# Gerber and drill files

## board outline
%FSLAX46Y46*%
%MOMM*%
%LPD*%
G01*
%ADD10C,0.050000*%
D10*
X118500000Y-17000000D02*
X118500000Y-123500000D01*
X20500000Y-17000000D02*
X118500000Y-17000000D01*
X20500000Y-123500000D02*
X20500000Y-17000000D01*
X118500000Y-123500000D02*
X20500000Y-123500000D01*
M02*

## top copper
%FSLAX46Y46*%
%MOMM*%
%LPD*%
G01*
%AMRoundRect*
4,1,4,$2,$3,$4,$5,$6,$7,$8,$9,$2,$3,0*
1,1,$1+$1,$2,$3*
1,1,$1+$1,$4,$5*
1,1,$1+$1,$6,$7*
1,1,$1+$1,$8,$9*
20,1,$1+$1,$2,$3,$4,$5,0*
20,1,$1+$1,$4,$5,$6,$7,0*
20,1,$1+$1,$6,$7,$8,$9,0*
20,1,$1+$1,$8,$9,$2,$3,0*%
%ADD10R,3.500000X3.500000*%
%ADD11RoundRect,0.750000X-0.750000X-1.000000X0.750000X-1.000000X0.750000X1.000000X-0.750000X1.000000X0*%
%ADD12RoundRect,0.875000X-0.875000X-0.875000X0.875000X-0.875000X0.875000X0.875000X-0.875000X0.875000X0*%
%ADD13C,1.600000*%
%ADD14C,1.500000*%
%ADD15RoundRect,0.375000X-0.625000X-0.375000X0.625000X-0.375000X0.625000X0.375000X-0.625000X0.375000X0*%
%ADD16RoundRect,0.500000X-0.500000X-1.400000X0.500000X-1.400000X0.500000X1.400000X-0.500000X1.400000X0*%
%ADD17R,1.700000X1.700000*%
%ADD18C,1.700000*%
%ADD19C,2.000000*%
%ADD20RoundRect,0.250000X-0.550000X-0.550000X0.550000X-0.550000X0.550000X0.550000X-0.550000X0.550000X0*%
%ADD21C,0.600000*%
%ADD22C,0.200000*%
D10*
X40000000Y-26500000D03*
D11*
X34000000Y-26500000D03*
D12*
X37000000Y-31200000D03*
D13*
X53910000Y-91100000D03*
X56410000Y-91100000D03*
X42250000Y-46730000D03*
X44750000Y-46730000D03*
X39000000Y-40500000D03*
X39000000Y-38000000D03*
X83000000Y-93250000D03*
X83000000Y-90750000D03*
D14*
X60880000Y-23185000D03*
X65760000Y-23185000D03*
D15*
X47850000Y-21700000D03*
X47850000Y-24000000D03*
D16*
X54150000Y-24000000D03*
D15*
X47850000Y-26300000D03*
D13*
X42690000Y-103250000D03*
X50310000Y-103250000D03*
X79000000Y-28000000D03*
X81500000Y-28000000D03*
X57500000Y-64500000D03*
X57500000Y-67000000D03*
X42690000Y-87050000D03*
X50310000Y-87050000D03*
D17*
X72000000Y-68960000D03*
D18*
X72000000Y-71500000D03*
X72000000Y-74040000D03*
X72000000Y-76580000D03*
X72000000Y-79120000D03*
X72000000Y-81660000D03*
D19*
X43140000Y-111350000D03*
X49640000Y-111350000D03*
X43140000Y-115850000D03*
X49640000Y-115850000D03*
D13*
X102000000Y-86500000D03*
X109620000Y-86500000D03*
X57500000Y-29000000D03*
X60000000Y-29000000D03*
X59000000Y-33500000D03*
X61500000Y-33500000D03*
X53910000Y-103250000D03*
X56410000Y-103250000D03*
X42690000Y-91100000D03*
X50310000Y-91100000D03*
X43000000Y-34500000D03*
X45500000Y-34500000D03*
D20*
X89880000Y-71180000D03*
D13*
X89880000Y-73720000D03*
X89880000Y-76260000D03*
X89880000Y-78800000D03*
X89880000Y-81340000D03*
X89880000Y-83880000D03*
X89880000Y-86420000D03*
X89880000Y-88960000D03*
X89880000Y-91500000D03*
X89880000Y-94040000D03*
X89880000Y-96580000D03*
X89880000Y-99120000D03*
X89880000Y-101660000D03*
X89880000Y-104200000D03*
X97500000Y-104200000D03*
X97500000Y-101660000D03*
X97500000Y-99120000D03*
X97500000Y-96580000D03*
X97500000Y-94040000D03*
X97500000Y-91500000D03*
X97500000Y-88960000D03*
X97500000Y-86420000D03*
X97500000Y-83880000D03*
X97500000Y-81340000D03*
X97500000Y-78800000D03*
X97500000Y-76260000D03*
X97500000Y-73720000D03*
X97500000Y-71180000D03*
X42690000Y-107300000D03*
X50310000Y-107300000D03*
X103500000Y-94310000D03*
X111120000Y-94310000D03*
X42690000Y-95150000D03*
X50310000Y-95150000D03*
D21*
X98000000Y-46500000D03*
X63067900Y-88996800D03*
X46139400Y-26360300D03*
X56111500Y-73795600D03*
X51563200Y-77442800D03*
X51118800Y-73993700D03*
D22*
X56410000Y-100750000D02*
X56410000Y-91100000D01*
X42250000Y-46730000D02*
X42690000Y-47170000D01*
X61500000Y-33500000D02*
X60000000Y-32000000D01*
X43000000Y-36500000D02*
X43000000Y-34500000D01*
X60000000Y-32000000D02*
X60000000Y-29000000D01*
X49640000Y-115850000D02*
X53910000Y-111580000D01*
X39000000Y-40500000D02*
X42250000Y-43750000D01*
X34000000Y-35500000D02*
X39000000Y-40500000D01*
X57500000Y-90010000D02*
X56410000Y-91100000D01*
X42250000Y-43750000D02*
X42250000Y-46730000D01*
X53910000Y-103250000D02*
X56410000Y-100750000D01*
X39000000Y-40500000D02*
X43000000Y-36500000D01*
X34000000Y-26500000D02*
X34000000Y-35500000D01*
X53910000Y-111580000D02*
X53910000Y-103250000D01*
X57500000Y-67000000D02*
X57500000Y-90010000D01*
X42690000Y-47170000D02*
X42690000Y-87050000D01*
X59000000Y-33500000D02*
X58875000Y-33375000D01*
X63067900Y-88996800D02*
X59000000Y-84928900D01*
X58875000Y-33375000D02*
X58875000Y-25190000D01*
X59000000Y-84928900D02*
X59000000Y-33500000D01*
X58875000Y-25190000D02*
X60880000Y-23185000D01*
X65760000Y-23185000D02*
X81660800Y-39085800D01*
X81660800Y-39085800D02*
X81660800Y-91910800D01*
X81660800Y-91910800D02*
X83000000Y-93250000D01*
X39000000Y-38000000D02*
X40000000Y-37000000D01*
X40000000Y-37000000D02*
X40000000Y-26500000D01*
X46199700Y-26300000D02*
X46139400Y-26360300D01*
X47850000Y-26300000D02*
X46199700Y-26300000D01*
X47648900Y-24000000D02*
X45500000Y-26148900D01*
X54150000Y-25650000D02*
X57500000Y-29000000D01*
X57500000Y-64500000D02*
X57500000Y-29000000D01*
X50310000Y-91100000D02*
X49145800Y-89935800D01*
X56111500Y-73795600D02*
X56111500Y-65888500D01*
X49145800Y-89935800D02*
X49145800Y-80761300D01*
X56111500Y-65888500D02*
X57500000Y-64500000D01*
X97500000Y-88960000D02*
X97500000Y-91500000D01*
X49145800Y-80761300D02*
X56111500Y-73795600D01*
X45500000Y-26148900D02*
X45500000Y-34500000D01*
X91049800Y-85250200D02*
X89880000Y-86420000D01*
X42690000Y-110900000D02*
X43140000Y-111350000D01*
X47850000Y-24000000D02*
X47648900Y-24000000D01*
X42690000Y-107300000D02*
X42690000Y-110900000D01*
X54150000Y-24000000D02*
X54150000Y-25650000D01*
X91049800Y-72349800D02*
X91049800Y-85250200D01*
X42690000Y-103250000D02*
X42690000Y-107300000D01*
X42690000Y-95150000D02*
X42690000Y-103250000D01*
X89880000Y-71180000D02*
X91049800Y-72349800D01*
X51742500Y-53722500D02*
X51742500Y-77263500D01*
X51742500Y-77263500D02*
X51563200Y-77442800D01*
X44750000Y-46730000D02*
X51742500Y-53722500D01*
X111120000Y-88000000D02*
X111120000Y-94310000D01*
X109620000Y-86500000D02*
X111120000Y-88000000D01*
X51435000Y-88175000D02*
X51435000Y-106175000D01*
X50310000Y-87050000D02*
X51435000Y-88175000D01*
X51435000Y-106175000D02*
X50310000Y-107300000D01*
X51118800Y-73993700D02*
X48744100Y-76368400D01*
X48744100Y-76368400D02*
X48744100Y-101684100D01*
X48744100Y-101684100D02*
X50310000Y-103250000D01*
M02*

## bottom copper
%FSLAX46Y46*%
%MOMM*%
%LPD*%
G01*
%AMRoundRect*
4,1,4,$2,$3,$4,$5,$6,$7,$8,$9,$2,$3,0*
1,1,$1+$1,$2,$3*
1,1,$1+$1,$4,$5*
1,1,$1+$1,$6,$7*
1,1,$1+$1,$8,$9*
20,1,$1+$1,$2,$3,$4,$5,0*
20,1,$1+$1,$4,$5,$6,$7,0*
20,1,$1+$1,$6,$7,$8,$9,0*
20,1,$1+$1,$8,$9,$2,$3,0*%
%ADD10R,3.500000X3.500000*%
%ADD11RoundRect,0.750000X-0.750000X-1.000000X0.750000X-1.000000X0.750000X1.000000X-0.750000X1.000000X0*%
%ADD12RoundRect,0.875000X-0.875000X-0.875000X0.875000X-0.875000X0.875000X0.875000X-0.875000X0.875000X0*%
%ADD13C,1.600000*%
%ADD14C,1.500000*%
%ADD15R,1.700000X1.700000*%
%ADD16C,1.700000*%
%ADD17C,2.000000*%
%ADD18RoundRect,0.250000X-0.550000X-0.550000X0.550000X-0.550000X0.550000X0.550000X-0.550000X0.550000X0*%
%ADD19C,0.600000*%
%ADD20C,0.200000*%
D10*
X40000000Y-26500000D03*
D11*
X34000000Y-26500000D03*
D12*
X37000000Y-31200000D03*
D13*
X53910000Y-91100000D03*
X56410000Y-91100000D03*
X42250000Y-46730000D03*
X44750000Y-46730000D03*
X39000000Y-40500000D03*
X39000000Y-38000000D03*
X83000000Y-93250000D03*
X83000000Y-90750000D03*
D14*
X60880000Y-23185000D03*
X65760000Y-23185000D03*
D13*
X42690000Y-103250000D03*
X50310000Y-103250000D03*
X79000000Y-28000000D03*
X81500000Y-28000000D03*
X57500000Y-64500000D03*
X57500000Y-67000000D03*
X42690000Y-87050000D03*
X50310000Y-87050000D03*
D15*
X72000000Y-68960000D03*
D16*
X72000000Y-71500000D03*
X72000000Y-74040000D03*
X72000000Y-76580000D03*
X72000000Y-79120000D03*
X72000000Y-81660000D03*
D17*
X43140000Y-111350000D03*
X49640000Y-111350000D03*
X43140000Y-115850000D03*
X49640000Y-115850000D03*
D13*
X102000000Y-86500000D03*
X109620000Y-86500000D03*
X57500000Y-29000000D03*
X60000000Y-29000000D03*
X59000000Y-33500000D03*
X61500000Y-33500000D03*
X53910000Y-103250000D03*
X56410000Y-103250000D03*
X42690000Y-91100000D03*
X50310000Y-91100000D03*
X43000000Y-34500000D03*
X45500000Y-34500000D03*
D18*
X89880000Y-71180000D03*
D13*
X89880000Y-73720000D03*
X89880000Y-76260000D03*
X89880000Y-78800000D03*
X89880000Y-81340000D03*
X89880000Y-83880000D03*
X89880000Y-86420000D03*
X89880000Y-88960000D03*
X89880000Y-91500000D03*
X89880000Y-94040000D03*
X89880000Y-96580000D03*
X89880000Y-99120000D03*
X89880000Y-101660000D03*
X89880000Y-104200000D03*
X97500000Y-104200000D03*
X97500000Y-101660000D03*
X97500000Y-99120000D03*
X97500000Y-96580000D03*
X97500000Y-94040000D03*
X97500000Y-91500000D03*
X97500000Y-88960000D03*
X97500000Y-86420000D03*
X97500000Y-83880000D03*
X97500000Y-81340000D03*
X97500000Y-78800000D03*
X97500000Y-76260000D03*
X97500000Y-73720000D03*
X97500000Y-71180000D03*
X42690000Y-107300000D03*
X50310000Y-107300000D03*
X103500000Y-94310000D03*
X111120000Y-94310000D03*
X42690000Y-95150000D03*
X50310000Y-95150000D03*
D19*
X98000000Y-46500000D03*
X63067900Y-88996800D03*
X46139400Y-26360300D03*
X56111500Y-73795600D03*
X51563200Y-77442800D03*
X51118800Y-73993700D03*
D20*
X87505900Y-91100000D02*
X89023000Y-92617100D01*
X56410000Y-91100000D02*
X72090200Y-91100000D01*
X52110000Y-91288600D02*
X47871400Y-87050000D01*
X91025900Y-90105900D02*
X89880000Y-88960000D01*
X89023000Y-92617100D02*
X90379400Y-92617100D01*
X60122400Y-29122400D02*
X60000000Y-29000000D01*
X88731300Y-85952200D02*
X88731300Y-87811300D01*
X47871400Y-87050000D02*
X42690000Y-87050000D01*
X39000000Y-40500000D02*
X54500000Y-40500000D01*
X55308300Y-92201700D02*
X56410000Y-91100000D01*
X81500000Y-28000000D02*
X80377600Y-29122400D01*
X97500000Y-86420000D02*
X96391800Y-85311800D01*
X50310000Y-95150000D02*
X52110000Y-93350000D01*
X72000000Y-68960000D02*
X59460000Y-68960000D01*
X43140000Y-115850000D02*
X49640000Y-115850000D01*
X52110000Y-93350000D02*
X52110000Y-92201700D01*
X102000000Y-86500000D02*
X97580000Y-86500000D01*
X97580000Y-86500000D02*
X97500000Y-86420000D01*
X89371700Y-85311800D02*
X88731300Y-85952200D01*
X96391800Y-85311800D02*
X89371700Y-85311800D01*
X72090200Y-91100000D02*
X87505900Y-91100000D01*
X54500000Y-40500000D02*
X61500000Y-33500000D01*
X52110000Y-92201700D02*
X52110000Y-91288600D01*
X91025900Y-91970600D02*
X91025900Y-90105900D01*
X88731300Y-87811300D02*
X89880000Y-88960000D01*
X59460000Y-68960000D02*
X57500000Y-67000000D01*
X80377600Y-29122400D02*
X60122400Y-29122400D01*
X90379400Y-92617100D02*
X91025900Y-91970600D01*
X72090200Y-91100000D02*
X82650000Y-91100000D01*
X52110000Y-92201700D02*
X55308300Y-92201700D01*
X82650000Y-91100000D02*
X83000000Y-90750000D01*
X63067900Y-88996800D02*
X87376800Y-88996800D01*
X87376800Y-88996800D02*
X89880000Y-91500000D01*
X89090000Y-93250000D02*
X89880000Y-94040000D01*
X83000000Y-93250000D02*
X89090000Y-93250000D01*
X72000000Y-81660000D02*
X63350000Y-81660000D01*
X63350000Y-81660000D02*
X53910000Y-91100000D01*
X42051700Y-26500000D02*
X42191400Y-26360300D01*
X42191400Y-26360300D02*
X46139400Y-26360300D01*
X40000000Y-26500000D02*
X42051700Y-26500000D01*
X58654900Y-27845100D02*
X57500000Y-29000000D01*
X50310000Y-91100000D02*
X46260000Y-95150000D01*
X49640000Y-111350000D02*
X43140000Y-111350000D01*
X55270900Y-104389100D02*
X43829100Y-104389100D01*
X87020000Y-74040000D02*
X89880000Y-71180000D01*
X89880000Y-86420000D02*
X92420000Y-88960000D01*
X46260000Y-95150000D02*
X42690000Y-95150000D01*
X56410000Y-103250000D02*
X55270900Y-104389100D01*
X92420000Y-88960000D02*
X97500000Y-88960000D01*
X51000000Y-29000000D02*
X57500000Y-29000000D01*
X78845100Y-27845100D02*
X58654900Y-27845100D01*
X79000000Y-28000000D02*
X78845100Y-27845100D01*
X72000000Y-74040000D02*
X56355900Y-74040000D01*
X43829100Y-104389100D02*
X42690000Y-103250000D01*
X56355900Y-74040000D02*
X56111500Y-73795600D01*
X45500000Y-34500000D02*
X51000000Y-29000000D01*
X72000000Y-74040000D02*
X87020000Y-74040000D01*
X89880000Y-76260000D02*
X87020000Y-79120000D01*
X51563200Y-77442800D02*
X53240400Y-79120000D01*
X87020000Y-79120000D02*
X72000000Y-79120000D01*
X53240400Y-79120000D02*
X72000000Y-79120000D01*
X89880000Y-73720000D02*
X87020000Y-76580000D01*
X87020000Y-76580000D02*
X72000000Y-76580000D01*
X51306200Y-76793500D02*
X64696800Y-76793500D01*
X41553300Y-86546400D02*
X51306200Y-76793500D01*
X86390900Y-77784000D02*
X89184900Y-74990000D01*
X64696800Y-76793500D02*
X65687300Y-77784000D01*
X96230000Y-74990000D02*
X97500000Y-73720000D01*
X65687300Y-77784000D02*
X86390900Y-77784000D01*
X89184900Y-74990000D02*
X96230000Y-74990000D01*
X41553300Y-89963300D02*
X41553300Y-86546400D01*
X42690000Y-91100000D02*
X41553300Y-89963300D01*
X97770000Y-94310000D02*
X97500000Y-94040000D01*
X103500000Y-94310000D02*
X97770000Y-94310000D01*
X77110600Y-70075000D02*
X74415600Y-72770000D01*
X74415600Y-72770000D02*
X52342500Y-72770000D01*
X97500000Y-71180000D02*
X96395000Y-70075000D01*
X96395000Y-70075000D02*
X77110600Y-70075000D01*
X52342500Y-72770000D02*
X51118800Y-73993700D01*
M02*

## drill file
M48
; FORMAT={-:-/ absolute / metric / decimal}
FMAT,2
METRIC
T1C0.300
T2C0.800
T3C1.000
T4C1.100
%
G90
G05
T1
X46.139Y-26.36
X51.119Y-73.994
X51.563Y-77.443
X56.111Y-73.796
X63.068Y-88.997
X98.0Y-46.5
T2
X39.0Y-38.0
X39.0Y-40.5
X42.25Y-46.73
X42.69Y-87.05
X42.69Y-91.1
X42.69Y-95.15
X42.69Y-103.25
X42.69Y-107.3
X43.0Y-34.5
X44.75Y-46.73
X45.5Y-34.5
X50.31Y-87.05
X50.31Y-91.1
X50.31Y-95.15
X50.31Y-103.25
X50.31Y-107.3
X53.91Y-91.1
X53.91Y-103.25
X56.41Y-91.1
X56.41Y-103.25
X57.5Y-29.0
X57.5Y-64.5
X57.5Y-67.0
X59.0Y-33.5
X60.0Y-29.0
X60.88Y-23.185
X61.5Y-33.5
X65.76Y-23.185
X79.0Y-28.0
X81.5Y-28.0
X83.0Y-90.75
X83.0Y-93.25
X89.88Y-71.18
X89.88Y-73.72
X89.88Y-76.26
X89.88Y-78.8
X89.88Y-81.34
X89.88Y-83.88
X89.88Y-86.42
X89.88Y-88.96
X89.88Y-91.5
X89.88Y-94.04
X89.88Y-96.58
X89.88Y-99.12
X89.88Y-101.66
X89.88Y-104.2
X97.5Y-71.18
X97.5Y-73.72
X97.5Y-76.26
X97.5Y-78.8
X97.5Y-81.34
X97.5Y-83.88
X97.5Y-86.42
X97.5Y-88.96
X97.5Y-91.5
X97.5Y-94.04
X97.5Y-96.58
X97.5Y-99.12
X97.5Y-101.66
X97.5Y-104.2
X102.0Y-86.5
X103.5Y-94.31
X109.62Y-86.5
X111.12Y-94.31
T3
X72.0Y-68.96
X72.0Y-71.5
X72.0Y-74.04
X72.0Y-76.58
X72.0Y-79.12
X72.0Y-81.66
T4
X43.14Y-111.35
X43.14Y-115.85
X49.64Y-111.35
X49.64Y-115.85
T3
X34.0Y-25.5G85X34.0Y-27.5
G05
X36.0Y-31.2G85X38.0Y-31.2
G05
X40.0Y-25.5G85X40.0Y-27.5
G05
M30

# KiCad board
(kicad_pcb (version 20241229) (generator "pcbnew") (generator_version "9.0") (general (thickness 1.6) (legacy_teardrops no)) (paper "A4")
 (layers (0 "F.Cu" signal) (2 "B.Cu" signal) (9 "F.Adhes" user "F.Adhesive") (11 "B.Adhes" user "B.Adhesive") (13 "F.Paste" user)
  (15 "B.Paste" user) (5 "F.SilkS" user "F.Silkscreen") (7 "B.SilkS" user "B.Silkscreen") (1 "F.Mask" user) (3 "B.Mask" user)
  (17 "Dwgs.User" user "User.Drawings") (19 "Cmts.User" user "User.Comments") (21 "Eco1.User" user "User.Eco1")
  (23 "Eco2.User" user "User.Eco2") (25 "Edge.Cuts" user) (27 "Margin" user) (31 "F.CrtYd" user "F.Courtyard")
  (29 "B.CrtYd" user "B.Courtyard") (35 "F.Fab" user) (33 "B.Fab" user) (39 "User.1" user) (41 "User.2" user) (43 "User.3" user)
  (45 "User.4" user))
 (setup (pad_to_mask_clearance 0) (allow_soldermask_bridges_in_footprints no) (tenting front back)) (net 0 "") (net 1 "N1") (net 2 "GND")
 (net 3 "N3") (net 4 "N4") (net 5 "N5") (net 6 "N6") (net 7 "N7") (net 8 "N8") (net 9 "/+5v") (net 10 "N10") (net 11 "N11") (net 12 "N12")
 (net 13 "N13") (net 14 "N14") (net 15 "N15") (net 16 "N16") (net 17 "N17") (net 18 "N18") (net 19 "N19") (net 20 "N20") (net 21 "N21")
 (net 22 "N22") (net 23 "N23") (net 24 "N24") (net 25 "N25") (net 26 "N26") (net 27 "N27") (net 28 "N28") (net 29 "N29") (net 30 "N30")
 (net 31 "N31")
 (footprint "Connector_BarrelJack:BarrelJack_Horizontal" (layer "F.Cu") (at 40 26.5)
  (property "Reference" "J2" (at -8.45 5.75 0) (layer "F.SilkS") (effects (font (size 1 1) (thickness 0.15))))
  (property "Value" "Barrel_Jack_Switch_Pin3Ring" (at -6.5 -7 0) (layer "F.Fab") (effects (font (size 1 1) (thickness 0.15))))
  (pad "1" thru_hole rect (at 0 0) (size 3.5 3.5) (drill oval 1 3) (layers "*.Cu" "*.Mask") (remove_unused_layers no) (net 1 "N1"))
  (pad "2" thru_hole roundrect (at -6 0) (size 3 3.5) (drill oval 1 3) (layers "*.Cu" "*.Mask") (remove_unused_layers no)
   (roundrect_rratio 0.25) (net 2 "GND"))
  (pad "3" thru_hole roundrect (at -3 4.7) (size 3.5 3.5) (drill oval 3 1) (layers "*.Cu" "*.Mask") (remove_unused_layers no)
   (roundrect_rratio 0.25) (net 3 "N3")))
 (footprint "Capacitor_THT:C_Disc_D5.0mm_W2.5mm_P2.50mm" (layer "F.Cu") (at 53.91 91.1)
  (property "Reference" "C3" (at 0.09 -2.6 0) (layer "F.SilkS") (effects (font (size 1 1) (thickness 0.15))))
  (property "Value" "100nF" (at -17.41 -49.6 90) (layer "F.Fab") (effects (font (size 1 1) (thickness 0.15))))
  (pad "1" thru_hole circle (at 0 0) (size 1.6 1.6) (drill 0.8) (layers "*.Cu" "*.Mask") (remove_unused_layers no) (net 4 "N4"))
  (pad "2" thru_hole circle (at 2.5 0) (size 1.6 1.6) (drill 0.8) (layers "*.Cu" "*.Mask") (remove_unused_layers no) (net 2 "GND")))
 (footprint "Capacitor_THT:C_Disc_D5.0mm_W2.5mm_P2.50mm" (layer "F.Cu") (at 42.25 46.73)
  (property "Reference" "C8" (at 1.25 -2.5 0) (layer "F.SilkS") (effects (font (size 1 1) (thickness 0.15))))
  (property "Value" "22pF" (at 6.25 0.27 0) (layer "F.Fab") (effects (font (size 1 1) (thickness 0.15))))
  (pad "1" thru_hole circle (at 0 0) (size 1.6 1.6) (drill 0.8) (layers "*.Cu" "*.Mask") (remove_unused_layers no) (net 2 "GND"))
  (pad "2" thru_hole circle (at 2.5 0) (size 1.6 1.6) (drill 0.8) (layers "*.Cu" "*.Mask") (remove_unused_layers no) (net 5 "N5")))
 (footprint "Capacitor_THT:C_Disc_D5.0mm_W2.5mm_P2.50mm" (layer "F.Cu") (at 39 40.5 90)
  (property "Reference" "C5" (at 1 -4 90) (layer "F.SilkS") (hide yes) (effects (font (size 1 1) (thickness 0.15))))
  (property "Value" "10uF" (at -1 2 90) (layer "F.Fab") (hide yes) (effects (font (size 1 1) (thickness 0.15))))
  (pad "1" thru_hole circle (at 0 0 90) (size 1.6 1.6) (drill 0.8) (layers "*.Cu" "*.Mask") (remove_unused_layers no) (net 2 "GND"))
  (pad "2" thru_hole circle (at 2.5 0 90) (size 1.6 1.6) (drill 0.8) (layers "*.Cu" "*.Mask") (remove_unused_layers no) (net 1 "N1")))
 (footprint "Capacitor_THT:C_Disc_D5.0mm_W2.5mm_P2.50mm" (layer "F.Cu") (at 83 93.25 90)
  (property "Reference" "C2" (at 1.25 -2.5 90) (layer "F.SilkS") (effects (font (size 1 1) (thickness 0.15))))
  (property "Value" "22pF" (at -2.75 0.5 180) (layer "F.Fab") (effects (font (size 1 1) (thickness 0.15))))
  (pad "1" thru_hole circle (at 0 0 90) (size 1.6 1.6) (drill 0.8) (layers "*.Cu" "*.Mask") (remove_unused_layers no) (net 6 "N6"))
  (pad "2" thru_hole circle (at 2.5 0 90) (size 1.6 1.6) (drill 0.8) (layers "*.Cu" "*.Mask") (remove_unused_layers no) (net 2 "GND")))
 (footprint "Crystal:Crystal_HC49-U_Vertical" (layer "F.Cu") (at 60.88 23.185)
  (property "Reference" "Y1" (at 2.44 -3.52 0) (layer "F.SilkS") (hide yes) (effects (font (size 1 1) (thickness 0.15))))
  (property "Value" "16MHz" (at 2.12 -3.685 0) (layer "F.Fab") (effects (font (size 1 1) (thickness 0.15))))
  (pad "1" thru_hole circle (at 0 0) (size 1.5 1.5) (drill 0.8) (layers "*.Cu" "*.Mask") (remove_unused_layers no) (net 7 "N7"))
  (pad "2" thru_hole circle (at 4.88 0) (size 1.5 1.5) (drill 0.8) (layers "*.Cu" "*.Mask") (remove_unused_layers no) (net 6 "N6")))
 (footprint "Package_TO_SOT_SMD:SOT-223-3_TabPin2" (layer "F.Cu") (at 51 24)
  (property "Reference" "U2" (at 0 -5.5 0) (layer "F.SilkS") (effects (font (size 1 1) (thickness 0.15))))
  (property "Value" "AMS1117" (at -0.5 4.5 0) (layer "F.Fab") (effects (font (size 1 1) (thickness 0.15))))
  (pad "1" smd roundrect (at -3.15 -2.3) (size 2 1.5) (layers "F.Cu" "F.Mask" "F.Paste") (roundrect_rratio 0.25) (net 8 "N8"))
  (pad "2" smd roundrect (at -3.15 0) (size 2 1.5) (layers "F.Cu" "F.Mask" "F.Paste") (roundrect_rratio 0.25) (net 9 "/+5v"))
  (pad "2" smd roundrect (at 3.15 0) (size 2 3.8) (layers "F.Cu" "F.Mask" "F.Paste") (roundrect_rratio 0.25) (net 9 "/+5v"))
  (pad "3" smd roundrect (at -3.15 2.3) (size 2 1.5) (layers "F.Cu" "F.Mask" "F.Paste") (roundrect_rratio 0.25) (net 1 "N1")))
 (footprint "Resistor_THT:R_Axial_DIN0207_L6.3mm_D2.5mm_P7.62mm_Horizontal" (layer "F.Cu") (at 42.69 103.25)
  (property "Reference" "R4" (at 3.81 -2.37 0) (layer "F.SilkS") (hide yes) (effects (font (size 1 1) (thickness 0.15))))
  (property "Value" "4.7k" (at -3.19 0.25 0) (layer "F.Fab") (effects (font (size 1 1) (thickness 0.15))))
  (pad "1" thru_hole circle (at 0 0) (size 1.6 1.6) (drill 0.8) (layers "*.Cu" "*.Mask") (remove_unused_layers no) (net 9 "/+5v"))
  (pad "2" thru_hole circle (at 7.62 0) (size 1.6 1.6) (drill 0.8) (layers "*.Cu" "*.Mask") (remove_unused_layers no) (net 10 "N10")))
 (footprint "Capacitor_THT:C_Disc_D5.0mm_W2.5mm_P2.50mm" (layer "F.Cu") (at 79 28)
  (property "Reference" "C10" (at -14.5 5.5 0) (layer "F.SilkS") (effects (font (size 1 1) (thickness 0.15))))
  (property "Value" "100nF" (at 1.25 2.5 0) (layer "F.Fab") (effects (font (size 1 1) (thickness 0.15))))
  (pad "1" thru_hole circle (at 0 0) (size 1.6 1.6) (drill 0.8) (layers "*.Cu" "*.Mask") (remove_unused_layers no) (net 9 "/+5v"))
  (pad "2" thru_hole circle (at 2.5 0) (size 1.6 1.6) (drill 0.8) (layers "*.Cu" "*.Mask") (remove_unused_layers no) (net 2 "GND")))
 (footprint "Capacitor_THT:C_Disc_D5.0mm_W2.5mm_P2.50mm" (layer "F.Cu") (at 57.5 64.5 -90)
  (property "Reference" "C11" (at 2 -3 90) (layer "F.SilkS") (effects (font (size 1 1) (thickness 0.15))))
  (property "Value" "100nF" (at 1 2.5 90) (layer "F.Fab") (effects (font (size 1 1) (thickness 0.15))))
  (pad "1" thru_hole circle (at 0 0 270) (size 1.6 1.6) (drill 0.8) (layers "*.Cu" "*.Mask") (remove_unused_layers no) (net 9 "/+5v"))
  (pad "2" thru_hole circle (at 2.5 0 270) (size 1.6 1.6) (drill 0.8) (layers "*.Cu" "*.Mask") (remove_unused_layers no) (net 2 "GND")))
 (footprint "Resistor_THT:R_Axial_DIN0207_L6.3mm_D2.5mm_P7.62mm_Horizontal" (layer "F.Cu") (at 42.69 87.05)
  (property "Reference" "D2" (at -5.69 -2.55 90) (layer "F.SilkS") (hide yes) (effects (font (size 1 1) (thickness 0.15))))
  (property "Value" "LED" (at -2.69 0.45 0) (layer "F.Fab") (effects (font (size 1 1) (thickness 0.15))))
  (pad "1" thru_hole circle (at 0 0) (size 1.6 1.6) (drill 0.8) (layers "*.Cu" "*.Mask") (remove_unused_layers no) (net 2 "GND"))
  (pad "2" thru_hole circle (at 7.62 0) (size 1.6 1.6) (drill 0.8) (layers "*.Cu" "*.Mask") (remove_unused_layers no) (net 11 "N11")))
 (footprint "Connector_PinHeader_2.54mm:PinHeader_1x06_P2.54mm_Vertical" (layer "F.Cu") (at 72 68.96)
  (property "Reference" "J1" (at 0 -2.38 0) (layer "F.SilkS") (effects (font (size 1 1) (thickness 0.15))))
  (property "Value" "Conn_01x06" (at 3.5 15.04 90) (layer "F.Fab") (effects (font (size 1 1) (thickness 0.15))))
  (pad "1" thru_hole rect (at 0 0) (size 1.7 1.7) (drill 1) (layers "*.Cu" "*.Mask") (remove_unused_layers no) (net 2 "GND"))
  (pad "2" thru_hole circle (at 0 2.54) (size 1.7 1.7) (drill 1) (layers "*.Cu" "*.Mask") (remove_unused_layers no) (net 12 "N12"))
  (pad "3" thru_hole circle (at 0 5.08) (size 1.7 1.7) (drill 1) (layers "*.Cu" "*.Mask") (remove_unused_layers no) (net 9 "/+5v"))
  (pad "4" thru_hole circle (at 0 7.62) (size 1.7 1.7) (drill 1) (layers "*.Cu" "*.Mask") (remove_unused_layers no) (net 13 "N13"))
  (pad "5" thru_hole circle (at 0 10.16) (size 1.7 1.7) (drill 1) (layers "*.Cu" "*.Mask") (remove_unused_layers no) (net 5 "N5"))
  (pad "6" thru_hole circle (at 0 12.7) (size 1.7 1.7) (drill 1) (layers "*.Cu" "*.Mask") (remove_unused_layers no) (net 4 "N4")))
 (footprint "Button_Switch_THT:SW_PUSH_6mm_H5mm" (layer "F.Cu") (at 43.14 111.35)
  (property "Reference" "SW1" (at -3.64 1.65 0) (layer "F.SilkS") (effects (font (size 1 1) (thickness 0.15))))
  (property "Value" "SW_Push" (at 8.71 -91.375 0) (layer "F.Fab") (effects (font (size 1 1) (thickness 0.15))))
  (pad "1" thru_hole circle (at 0 0 90) (size 2 2) (drill 1.1) (layers "*.Cu" "*.Mask") (remove_unused_layers no) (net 9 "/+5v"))
  (pad "1" thru_hole circle (at 6.5 0 90) (size 2 2) (drill 1.1) (layers "*.Cu" "*.Mask") (remove_unused_layers no) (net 9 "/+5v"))
  (pad "2" thru_hole circle (at 0 4.5 90) (size 2 2) (drill 1.1) (layers "*.Cu" "*.Mask") (remove_unused_layers no) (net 2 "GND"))
  (pad "2" thru_hole circle (at 6.5 4.5 90) (size 2 2) (drill 1.1) (layers "*.Cu" "*.Mask") (remove_unused_layers no) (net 2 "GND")))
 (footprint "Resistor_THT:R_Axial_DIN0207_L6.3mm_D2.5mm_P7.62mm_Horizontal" (layer "F.Cu") (at 102 86.5)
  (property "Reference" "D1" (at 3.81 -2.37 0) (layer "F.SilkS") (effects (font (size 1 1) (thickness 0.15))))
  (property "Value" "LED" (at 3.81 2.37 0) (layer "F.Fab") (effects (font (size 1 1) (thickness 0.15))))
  (pad "1" thru_hole circle (at 0 0) (size 1.6 1.6) (drill 0.8) (layers "*.Cu" "*.Mask") (remove_unused_layers no) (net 2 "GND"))
  (pad "2" thru_hole circle (at 7.62 0) (size 1.6 1.6) (drill 0.8) (layers "*.Cu" "*.Mask") (remove_unused_layers no) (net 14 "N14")))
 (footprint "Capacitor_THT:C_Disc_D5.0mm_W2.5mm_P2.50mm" (layer "F.Cu") (at 57.5 29)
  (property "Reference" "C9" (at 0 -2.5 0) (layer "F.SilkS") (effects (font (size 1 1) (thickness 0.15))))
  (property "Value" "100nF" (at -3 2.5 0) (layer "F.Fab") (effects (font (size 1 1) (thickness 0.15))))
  (pad "1" thru_hole circle (at 0 0) (size 1.6 1.6) (drill 0.8) (layers "*.Cu" "*.Mask") (remove_unused_layers no) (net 9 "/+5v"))
  (pad "2" thru_hole circle (at 2.5 0) (size 1.6 1.6) (drill 0.8) (layers "*.Cu" "*.Mask") (remove_unused_layers no) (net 2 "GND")))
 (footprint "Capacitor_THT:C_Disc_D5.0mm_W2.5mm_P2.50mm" (layer "F.Cu") (at 59 33.5)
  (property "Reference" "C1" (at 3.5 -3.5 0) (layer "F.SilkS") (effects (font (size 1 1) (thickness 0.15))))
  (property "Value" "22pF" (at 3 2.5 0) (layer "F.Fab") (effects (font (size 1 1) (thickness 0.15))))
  (pad "1" thru_hole circle (at 0 0) (size 1.6 1.6) (drill 0.8) (layers "*.Cu" "*.Mask") (remove_unused_layers no) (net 7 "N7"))
  (pad "2" thru_hole circle (at 2.5 0) (size 1.6 1.6) (drill 0.8) (layers "*.Cu" "*.Mask") (remove_unused_layers no) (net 2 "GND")))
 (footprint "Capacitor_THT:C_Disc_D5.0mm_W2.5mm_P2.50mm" (layer "F.Cu") (at 53.91 103.25)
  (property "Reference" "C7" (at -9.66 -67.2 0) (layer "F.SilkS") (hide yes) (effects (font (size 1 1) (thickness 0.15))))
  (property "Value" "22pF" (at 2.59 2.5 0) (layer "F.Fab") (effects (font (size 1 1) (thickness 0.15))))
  (pad "1" thru_hole circle (at 0 0) (size 1.6 1.6) (drill 0.8) (layers "*.Cu" "*.Mask") (remove_unused_layers no) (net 2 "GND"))
  (pad "2" thru_hole circle (at 2.5 0) (size 1.6 1.6) (drill 0.8) (layers "*.Cu" "*.Mask") (remove_unused_layers no) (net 9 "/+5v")))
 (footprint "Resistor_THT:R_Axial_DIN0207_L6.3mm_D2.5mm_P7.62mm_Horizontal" (layer "F.Cu") (at 42.69 91.1)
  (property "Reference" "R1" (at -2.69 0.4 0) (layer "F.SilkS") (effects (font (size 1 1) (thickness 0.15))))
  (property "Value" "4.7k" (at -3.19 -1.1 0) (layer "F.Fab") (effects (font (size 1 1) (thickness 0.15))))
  (pad "1" thru_hole circle (at 0 0) (size 1.6 1.6) (drill 0.8) (layers "*.Cu" "*.Mask") (remove_unused_layers no) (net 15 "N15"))
  (pad "2" thru_hole circle (at 7.62 0) (size 1.6 1.6) (drill 0.8) (layers "*.Cu" "*.Mask") (remove_unused_layers no) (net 9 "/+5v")))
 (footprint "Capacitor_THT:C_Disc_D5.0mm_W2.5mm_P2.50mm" (layer "F.Cu") (at 43 34.5)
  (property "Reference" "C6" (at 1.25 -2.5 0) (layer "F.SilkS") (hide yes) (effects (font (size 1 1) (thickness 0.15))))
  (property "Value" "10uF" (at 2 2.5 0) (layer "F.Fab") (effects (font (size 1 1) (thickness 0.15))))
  (pad "1" thru_hole circle (at 0 0) (size 1.6 1.6) (drill 0.8) (layers "*.Cu" "*.Mask") (remove_unused_layers no) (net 2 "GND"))
  (pad "2" thru_hole circle (at 2.5 0) (size 1.6 1.6) (drill 0.8) (layers "*.Cu" "*.Mask") (remove_unused_layers no) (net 9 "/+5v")))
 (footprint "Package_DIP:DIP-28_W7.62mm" (layer "F.Cu") (at 89.88 71.18)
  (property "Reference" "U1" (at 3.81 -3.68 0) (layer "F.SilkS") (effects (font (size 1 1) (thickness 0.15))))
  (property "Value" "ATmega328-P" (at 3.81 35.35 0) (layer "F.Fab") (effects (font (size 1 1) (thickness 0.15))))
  (pad "1" thru_hole roundrect (at 0 0) (size 1.6 1.6) (drill 0.8) (layers "*.Cu" "*.Mask") (remove_unused_layers no)
   (roundrect_rratio 0.15625) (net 9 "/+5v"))
  (pad "2" thru_hole circle (at 0 2.54) (size 1.6 1.6) (drill 0.8) (layers "*.Cu" "*.Mask") (remove_unused_layers no) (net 13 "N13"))
  (pad "3" thru_hole circle (at 0 5.08) (size 1.6 1.6) (drill 0.8) (layers "*.Cu" "*.Mask") (remove_unused_layers no) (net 5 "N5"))
  (pad "4" thru_hole circle (at 0 7.62) (size 1.6 1.6) (drill 0.8) (layers "*.Cu" "*.Mask") (remove_unused_layers no) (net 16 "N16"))
  (pad "5" thru_hole circle (at 0 10.16) (size 1.6 1.6) (drill 0.8) (layers "*.Cu" "*.Mask") (remove_unused_layers no) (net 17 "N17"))
  (pad "6" thru_hole circle (at 0 12.7) (size 1.6 1.6) (drill 0.8) (layers "*.Cu" "*.Mask") (remove_unused_layers no) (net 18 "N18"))
  (pad "7" thru_hole circle (at 0 15.24) (size 1.6 1.6) (drill 0.8) (layers "*.Cu" "*.Mask") (remove_unused_layers no) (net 9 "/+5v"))
  (pad "8" thru_hole circle (at 0 17.78) (size 1.6 1.6) (drill 0.8) (layers "*.Cu" "*.Mask") (remove_unused_layers no) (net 2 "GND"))
  (pad "9" thru_hole circle (at 0 20.32) (size 1.6 1.6) (drill 0.8) (layers "*.Cu" "*.Mask") (remove_unused_layers no) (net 7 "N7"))
  (pad "10" thru_hole circle (at 0 22.86) (size 1.6 1.6) (drill 0.8) (layers "*.Cu" "*.Mask") (remove_unused_layers no) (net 6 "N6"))
  (pad "11" thru_hole circle (at 0 25.4) (size 1.6 1.6) (drill 0.8) (layers "*.Cu" "*.Mask") (remove_unused_layers no) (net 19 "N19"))
  (pad "12" thru_hole circle (at 0 27.94) (size 1.6 1.6) (drill 0.8) (layers "*.Cu" "*.Mask") (remove_unused_layers no) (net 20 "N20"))
  (pad "13" thru_hole circle (at 0 30.48) (size 1.6 1.6) (drill 0.8) (layers "*.Cu" "*.Mask") (remove_unused_layers no) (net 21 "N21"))
  (pad "14" thru_hole circle (at 0 33.02) (size 1.6 1.6) (drill 0.8) (layers "*.Cu" "*.Mask") (remove_unused_layers no) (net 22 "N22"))
  (pad "15" thru_hole circle (at 7.62 33.02) (size 1.6 1.6) (drill 0.8) (layers "*.Cu" "*.Mask") (remove_unused_layers no) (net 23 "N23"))
  (pad "16" thru_hole circle (at 7.62 30.48) (size 1.6 1.6) (drill 0.8) (layers "*.Cu" "*.Mask") (remove_unused_layers no) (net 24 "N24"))
  (pad "17" thru_hole circle (at 7.62 27.94) (size 1.6 1.6) (drill 0.8) (layers "*.Cu" "*.Mask") (remove_unused_layers no) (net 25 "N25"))
  (pad "18" thru_hole circle (at 7.62 25.4) (size 1.6 1.6) (drill 0.8) (layers "*.Cu" "*.Mask") (remove_unused_layers no) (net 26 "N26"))
  (pad "19" thru_hole circle (at 7.62 22.86) (size 1.6 1.6) (drill 0.8) (layers "*.Cu" "*.Mask") (remove_unused_layers no) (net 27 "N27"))
  (pad "20" thru_hole circle (at 7.62 20.32) (size 1.6 1.6) (drill 0.8) (layers "*.Cu" "*.Mask") (remove_unused_layers no) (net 9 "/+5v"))
  (pad "21" thru_hole circle (at 7.62 17.78) (size 1.6 1.6) (drill 0.8) (layers "*.Cu" "*.Mask") (remove_unused_layers no) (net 9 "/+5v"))
  (pad "22" thru_hole circle (at 7.62 15.24) (size 1.6 1.6) (drill 0.8) (layers "*.Cu" "*.Mask") (remove_unused_layers no) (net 2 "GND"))
  (pad "23" thru_hole circle (at 7.62 12.7) (size 1.6 1.6) (drill 0.8) (layers "*.Cu" "*.Mask") (remove_unused_layers no) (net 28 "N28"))
  (pad "24" thru_hole circle (at 7.62 10.16) (size 1.6 1.6) (drill 0.8) (layers "*.Cu" "*.Mask") (remove_unused_layers no) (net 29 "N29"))
  (pad "25" thru_hole circle (at 7.62 7.62) (size 1.6 1.6) (drill 0.8) (layers "*.Cu" "*.Mask") (remove_unused_layers no) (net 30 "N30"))
  (pad "26" thru_hole circle (at 7.62 5.08) (size 1.6 1.6) (drill 0.8) (layers "*.Cu" "*.Mask") (remove_unused_layers no) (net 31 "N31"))
  (pad "27" thru_hole circle (at 7.62 2.54) (size 1.6 1.6) (drill 0.8) (layers "*.Cu" "*.Mask") (remove_unused_layers no) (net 15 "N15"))
  (pad "28" thru_hole circle (at 7.62 0) (size 1.6 1.6) (drill 0.8) (layers "*.Cu" "*.Mask") (remove_unused_layers no) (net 10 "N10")))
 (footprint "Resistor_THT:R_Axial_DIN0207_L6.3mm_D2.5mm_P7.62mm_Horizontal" (layer "F.Cu") (at 42.69 107.3)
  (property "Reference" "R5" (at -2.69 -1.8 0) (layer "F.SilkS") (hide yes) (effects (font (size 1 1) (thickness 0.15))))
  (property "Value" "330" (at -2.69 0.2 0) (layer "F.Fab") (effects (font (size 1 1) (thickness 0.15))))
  (pad "1" thru_hole circle (at 0 0) (size 1.6 1.6) (drill 0.8) (layers "*.Cu" "*.Mask") (remove_unused_layers no) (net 9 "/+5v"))
  (pad "2" thru_hole circle (at 7.62 0) (size 1.6 1.6) (drill 0.8) (layers "*.Cu" "*.Mask") (remove_unused_layers no) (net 11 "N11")))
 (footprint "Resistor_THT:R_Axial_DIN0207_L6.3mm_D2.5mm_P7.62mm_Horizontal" (layer "F.Cu") (at 103.5 94.31)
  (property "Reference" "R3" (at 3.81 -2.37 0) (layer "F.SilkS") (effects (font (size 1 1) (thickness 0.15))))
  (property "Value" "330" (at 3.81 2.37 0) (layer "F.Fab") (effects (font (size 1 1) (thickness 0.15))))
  (pad "1" thru_hole circle (at 0 0) (size 1.6 1.6) (drill 0.8) (layers "*.Cu" "*.Mask") (remove_unused_layers no) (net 27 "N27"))
  (pad "2" thru_hole circle (at 7.62 0) (size 1.6 1.6) (drill 0.8) (layers "*.Cu" "*.Mask") (remove_unused_layers no) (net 14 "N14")))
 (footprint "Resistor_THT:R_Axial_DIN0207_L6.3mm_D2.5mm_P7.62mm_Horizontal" (layer "F.Cu") (at 42.69 95.15)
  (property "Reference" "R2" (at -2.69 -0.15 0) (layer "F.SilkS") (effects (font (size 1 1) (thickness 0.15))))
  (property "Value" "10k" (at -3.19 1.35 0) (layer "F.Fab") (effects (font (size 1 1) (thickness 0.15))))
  (pad "1" thru_hole circle (at 0 0) (size 1.6 1.6) (drill 0.8) (layers "*.Cu" "*.Mask") (remove_unused_layers no) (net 9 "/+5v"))
  (pad "2" thru_hole circle (at 7.62 0) (size 1.6 1.6) (drill 0.8) (layers "*.Cu" "*.Mask") (remove_unused_layers no) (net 2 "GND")))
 (gr_line (start 118.5 17) (end 118.5 123.5) (stroke (width 0.05) (type default)) (layer "Edge.Cuts"))
 (gr_line (start 20.5 17) (end 118.5 17) (stroke (width 0.05) (type default)) (layer "Edge.Cuts"))
 (gr_line (start 20.5 123.5) (end 20.5 17) (stroke (width 0.05) (type default)) (layer "Edge.Cuts"))
 (gr_line (start 118.5 123.5) (end 20.5 123.5) (stroke (width 0.05) (type default)) (layer "Edge.Cuts"))
 (via (at 98 46.5) (size 0.6) (drill 0.3) (layers "F.Cu" "B.Cu") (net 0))
 (segment (start 56.41 100.75) (end 56.41 91.1) (width 0.2) (layer "F.Cu") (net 2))
 (segment (start 42.25 46.73) (end 42.69 47.17) (width 0.2) (layer "F.Cu") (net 2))
 (segment (start 61.5 33.5) (end 60 32) (width 0.2) (layer "F.Cu") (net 2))
 (segment (start 43 36.5) (end 43 34.5) (width 0.2) (layer "F.Cu") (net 2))
 (segment (start 60 32) (end 60 29) (width 0.2) (layer "F.Cu") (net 2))
 (segment (start 49.64 115.85) (end 53.91 111.58) (width 0.2) (layer "F.Cu") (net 2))
 (segment (start 39 40.5) (end 42.25 43.75) (width 0.2) (layer "F.Cu") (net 2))
 (segment (start 34 35.5) (end 39 40.5) (width 0.2) (layer "F.Cu") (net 2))
 (segment (start 57.5 90.01) (end 56.41 91.1) (width 0.2) (layer "F.Cu") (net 2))
 (segment (start 42.25 43.75) (end 42.25 46.73) (width 0.2) (layer "F.Cu") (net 2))
 (segment (start 53.91 103.25) (end 56.41 100.75) (width 0.2) (layer "F.Cu") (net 2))
 (segment (start 39 40.5) (end 43 36.5) (width 0.2) (layer "F.Cu") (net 2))
 (segment (start 34 26.5) (end 34 35.5) (width 0.2) (layer "F.Cu") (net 2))
 (segment (start 53.91 111.58) (end 53.91 103.25) (width 0.2) (layer "F.Cu") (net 2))
 (segment (start 57.5 67) (end 57.5 90.01) (width 0.2) (layer "F.Cu") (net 2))
 (segment (start 42.69 47.17) (end 42.69 87.05) (width 0.2) (layer "F.Cu") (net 2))
 (segment (start 87.5059 91.1) (end 89.023 92.6171) (width 0.2) (layer "B.Cu") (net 2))
 (segment (start 56.41 91.1) (end 72.0902 91.1) (width 0.2) (layer "B.Cu") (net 2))
 (segment (start 52.11 91.2886) (end 47.8714 87.05) (width 0.2) (layer "B.Cu") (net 2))
 (segment (start 91.0259 90.1059) (end 89.88 88.96) (width 0.2) (layer "B.Cu") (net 2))
 (segment (start 89.023 92.6171) (end 90.3794 92.6171) (width 0.2) (layer "B.Cu") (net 2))
 (segment (start 60.1224 29.1224) (end 60 29) (width 0.2) (layer "B.Cu") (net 2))
 (segment (start 88.7313 85.9522) (end 88.7313 87.8113) (width 0.2) (layer "B.Cu") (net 2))
 (segment (start 47.8714 87.05) (end 42.69 87.05) (width 0.2) (layer "B.Cu") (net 2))
 (segment (start 39 40.5) (end 54.5 40.5) (width 0.2) (layer "B.Cu") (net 2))
 (segment (start 55.3083 92.2017) (end 56.41 91.1) (width 0.2) (layer "B.Cu") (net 2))
 (segment (start 81.5 28) (end 80.3776 29.1224) (width 0.2) (layer "B.Cu") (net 2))
 (segment (start 97.5 86.42) (end 96.3918 85.3118) (width 0.2) (layer "B.Cu") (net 2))
 (segment (start 50.31 95.15) (end 52.11 93.35) (width 0.2) (layer "B.Cu") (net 2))
 (segment (start 72 68.96) (end 59.46 68.96) (width 0.2) (layer "B.Cu") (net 2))
 (segment (start 43.14 115.85) (end 49.64 115.85) (width 0.2) (layer "B.Cu") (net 2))
 (segment (start 52.11 93.35) (end 52.11 92.2017) (width 0.2) (layer "B.Cu") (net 2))
 (segment (start 102 86.5) (end 97.58 86.5) (width 0.2) (layer "B.Cu") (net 2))
 (segment (start 97.58 86.5) (end 97.5 86.42) (width 0.2) (layer "B.Cu") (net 2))
 (segment (start 89.3717 85.3118) (end 88.7313 85.9522) (width 0.2) (layer "B.Cu") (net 2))
 (segment (start 96.3918 85.3118) (end 89.3717 85.3118) (width 0.2) (layer "B.Cu") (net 2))
 (segment (start 72.0902 91.1) (end 87.5059 91.1) (width 0.2) (layer "B.Cu") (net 2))
 (segment (start 54.5 40.5) (end 61.5 33.5) (width 0.2) (layer "B.Cu") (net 2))
 (segment (start 52.11 92.2017) (end 52.11 91.2886) (width 0.2) (layer "B.Cu") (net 2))
 (segment (start 91.0259 91.9706) (end 91.0259 90.1059) (width 0.2) (layer "B.Cu") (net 2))
 (segment (start 88.7313 87.8113) (end 89.88 88.96) (width 0.2) (layer "B.Cu") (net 2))
 (segment (start 59.46 68.96) (end 57.5 67) (width 0.2) (layer "B.Cu") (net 2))
 (segment (start 80.3776 29.1224) (end 60.1224 29.1224) (width 0.2) (layer "B.Cu") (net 2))
 (segment (start 90.3794 92.6171) (end 91.0259 91.9706) (width 0.2) (layer "B.Cu") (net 2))
 (segment (start 72.0902 91.1) (end 82.65 91.1) (width 0.2) (layer "B.Cu") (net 2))
 (segment (start 52.11 92.2017) (end 55.3083 92.2017) (width 0.2) (layer "B.Cu") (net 2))
 (segment (start 82.65 91.1) (end 83 90.75) (width 0.2) (layer "B.Cu") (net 2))
 (segment (start 59 33.5) (end 58.875 33.375) (width 0.2) (layer "F.Cu") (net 7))
 (segment (start 63.0679 88.9968) (end 59 84.9289) (width 0.2) (layer "F.Cu") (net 7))
 (segment (start 58.875 33.375) (end 58.875 25.19) (width 0.2) (layer "F.Cu") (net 7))
 (segment (start 59 84.9289) (end 59 33.5) (width 0.2) (layer "F.Cu") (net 7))
 (segment (start 58.875 25.19) (end 60.88 23.185) (width 0.2) (layer "F.Cu") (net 7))
 (via (at 63.0679 88.9968) (size 0.6) (drill 0.3) (layers "F.Cu" "B.Cu") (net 7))
 (segment (start 63.0679 88.9968) (end 87.3768 88.9968) (width 0.2) (layer "B.Cu") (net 7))
 (segment (start 87.3768 88.9968) (end 89.88 91.5) (width 0.2) (layer "B.Cu") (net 7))
 (segment (start 65.76 23.185) (end 81.6608 39.0858) (width 0.2) (layer "F.Cu") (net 6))
 (segment (start 81.6608 39.0858) (end 81.6608 91.9108) (width 0.2) (layer "F.Cu") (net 6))
 (segment (start 81.6608 91.9108) (end 83 93.25) (width 0.2) (layer "F.Cu") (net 6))
 (segment (start 89.09 93.25) (end 89.88 94.04) (width 0.2) (layer "B.Cu") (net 6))
 (segment (start 83 93.25) (end 89.09 93.25) (width 0.2) (layer "B.Cu") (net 6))
 (segment (start 72 81.66) (end 63.35 81.66) (width 0.2) (layer "B.Cu") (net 4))
 (segment (start 63.35 81.66) (end 53.91 91.1) (width 0.2) (layer "B.Cu") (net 4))
 (segment (start 39 38) (end 40 37) (width 0.2) (layer "F.Cu") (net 1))
 (segment (start 40 37) (end 40 26.5) (width 0.2) (layer "F.Cu") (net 1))
 (segment (start 46.1997 26.3) (end 46.1394 26.3603) (width 0.2) (layer "F.Cu") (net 1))
 (segment (start 47.85 26.3) (end 46.1997 26.3) (width 0.2) (layer "F.Cu") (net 1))
 (via (at 46.1394 26.3603) (size 0.6) (drill 0.3) (layers "F.Cu" "B.Cu") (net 1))
 (segment (start 42.0517 26.5) (end 42.1914 26.3603) (width 0.2) (layer "B.Cu") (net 1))
 (segment (start 42.1914 26.3603) (end 46.1394 26.3603) (width 0.2) (layer "B.Cu") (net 1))
 (segment (start 40 26.5) (end 42.0517 26.5) (width 0.2) (layer "B.Cu") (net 1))
 (segment (start 47.6489 24) (end 45.5 26.1489) (width 0.2) (layer "F.Cu") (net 9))
 (segment (start 54.15 25.65) (end 57.5 29) (width 0.2) (layer "F.Cu") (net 9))
 (segment (start 57.5 64.5) (end 57.5 29) (width 0.2) (layer "F.Cu") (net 9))
 (segment (start 50.31 91.1) (end 49.1458 89.9358) (width 0.2) (layer "F.Cu") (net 9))
 (segment (start 56.1115 73.7956) (end 56.1115 65.8885) (width 0.2) (layer "F.Cu") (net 9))
 (segment (start 49.1458 89.9358) (end 49.1458 80.7613) (width 0.2) (layer "F.Cu") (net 9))
 (segment (start 56.1115 65.8885) (end 57.5 64.5) (width 0.2) (layer "F.Cu") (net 9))
 (segment (start 97.5 88.96) (end 97.5 91.5) (width 0.2) (layer "F.Cu") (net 9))
 (segment (start 49.1458 80.7613) (end 56.1115 73.7956) (width 0.2) (layer "F.Cu") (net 9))
 (segment (start 45.5 26.1489) (end 45.5 34.5) (width 0.2) (layer "F.Cu") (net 9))
 (segment (start 91.0498 85.2502) (end 89.88 86.42) (width 0.2) (layer "F.Cu") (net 9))
 (segment (start 42.69 110.9) (end 43.14 111.35) (width 0.2) (layer "F.Cu") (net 9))
 (segment (start 47.85 24) (end 47.6489 24) (width 0.2) (layer "F.Cu") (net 9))
 (segment (start 42.69 107.3) (end 42.69 110.9) (width 0.2) (layer "F.Cu") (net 9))
 (segment (start 54.15 24) (end 54.15 25.65) (width 0.2) (layer "F.Cu") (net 9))
 (segment (start 91.0498 72.3498) (end 91.0498 85.2502) (width 0.2) (layer "F.Cu") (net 9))
 (segment (start 42.69 103.25) (end 42.69 107.3) (width 0.2) (layer "F.Cu") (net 9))
 (segment (start 42.69 95.15) (end 42.69 103.25) (width 0.2) (layer "F.Cu") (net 9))
 (segment (start 89.88 71.18) (end 91.0498 72.3498) (width 0.2) (layer "F.Cu") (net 9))
 (via (at 56.1115 73.7956) (size 0.6) (drill 0.3) (layers "F.Cu" "B.Cu") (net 9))
 (segment (start 58.6549 27.8451) (end 57.5 29) (width 0.2) (layer "B.Cu") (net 9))
 (segment (start 50.31 91.1) (end 46.26 95.15) (width 0.2) (layer "B.Cu") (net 9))
 (segment (start 49.64 111.35) (end 43.14 111.35) (width 0.2) (layer "B.Cu") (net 9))
 (segment (start 55.2709 104.3891) (end 43.8291 104.3891) (width 0.2) (layer "B.Cu") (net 9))
 (segment (start 87.02 74.04) (end 89.88 71.18) (width 0.2) (layer "B.Cu") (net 9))
 (segment (start 89.88 86.42) (end 92.42 88.96) (width 0.2) (layer "B.Cu") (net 9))
 (segment (start 46.26 95.15) (end 42.69 95.15) (width 0.2) (layer "B.Cu") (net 9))
 (segment (start 56.41 103.25) (end 55.2709 104.3891) (width 0.2) (layer "B.Cu") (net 9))
 (segment (start 92.42 88.96) (end 97.5 88.96) (width 0.2) (layer "B.Cu") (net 9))
 (segment (start 51 29) (end 57.5 29) (width 0.2) (layer "B.Cu") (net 9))
 (segment (start 78.8451 27.8451) (end 58.6549 27.8451) (width 0.2) (layer "B.Cu") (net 9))
 (segment (start 79 28) (end 78.8451 27.8451) (width 0.2) (layer "B.Cu") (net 9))
 (segment (start 72 74.04) (end 56.3559 74.04) (width 0.2) (layer "B.Cu") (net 9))
 (segment (start 43.8291 104.3891) (end 42.69 103.25) (width 0.2) (layer "B.Cu") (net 9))
 (segment (start 56.3559 74.04) (end 56.1115 73.7956) (width 0.2) (layer "B.Cu") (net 9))
 (segment (start 45.5 34.5) (end 51 29) (width 0.2) (layer "B.Cu") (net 9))
 (segment (start 72 74.04) (end 87.02 74.04) (width 0.2) (layer "B.Cu") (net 9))
 (segment (start 51.7425 53.7225) (end 51.7425 77.2635) (width 0.2) (layer "F.Cu") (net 5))
 (segment (start 51.7425 77.2635) (end 51.5632 77.4428) (width 0.2) (layer "F.Cu") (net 5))
 (segment (start 44.75 46.73) (end 51.7425 53.7225) (width 0.2) (layer "F.Cu") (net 5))
 (via (at 51.5632 77.4428) (size 0.6) (drill 0.3) (layers "F.Cu" "B.Cu") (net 5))
 (segment (start 89.88 76.26) (end 87.02 79.12) (width 0.2) (layer "B.Cu") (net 5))
 (segment (start 51.5632 77.4428) (end 53.2404 79.12) (width 0.2) (layer "B.Cu") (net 5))
 (segment (start 87.02 79.12) (end 72 79.12) (width 0.2) (layer "B.Cu") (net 5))
 (segment (start 53.2404 79.12) (end 72 79.12) (width 0.2) (layer "B.Cu") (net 5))
 (segment (start 111.12 88) (end 111.12 94.31) (width 0.2) (layer "F.Cu") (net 14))
 (segment (start 109.62 86.5) (end 111.12 88) (width 0.2) (layer "F.Cu") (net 14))
 (segment (start 51.435 88.175) (end 51.435 106.175) (width 0.2) (layer "F.Cu") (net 11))
 (segment (start 50.31 87.05) (end 51.435 88.175) (width 0.2) (layer "F.Cu") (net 11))
 (segment (start 51.435 106.175) (end 50.31 107.3) (width 0.2) (layer "F.Cu") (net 11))
 (segment (start 89.88 73.72) (end 87.02 76.58) (width 0.2) (layer "B.Cu") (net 13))
 (segment (start 87.02 76.58) (end 72 76.58) (width 0.2) (layer "B.Cu") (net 13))
 (segment (start 51.3062 76.7935) (end 64.6968 76.7935) (width 0.2) (layer "B.Cu") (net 15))
 (segment (start 41.5533 86.5464) (end 51.3062 76.7935) (width 0.2) (layer "B.Cu") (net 15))
 (segment (start 86.3909 77.784) (end 89.1849 74.99) (width 0.2) (layer "B.Cu") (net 15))
 (segment (start 64.6968 76.7935) (end 65.6873 77.784) (width 0.2) (layer "B.Cu") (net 15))
 (segment (start 96.23 74.99) (end 97.5 73.72) (width 0.2) (layer "B.Cu") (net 15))
 (segment (start 65.6873 77.784) (end 86.3909 77.784) (width 0.2) (layer "B.Cu") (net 15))
 (segment (start 89.1849 74.99) (end 96.23 74.99) (width 0.2) (layer "B.Cu") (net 15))
 (segment (start 41.5533 89.9633) (end 41.5533 86.5464) (width 0.2) (layer "B.Cu") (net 15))
 (segment (start 42.69 91.1) (end 41.5533 89.9633) (width 0.2) (layer "B.Cu") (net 15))
 (segment (start 97.77 94.31) (end 97.5 94.04) (width 0.2) (layer "B.Cu") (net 27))
 (segment (start 103.5 94.31) (end 97.77 94.31) (width 0.2) (layer "B.Cu") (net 27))
 (segment (start 51.1188 73.9937) (end 48.7441 76.3684) (width 0.2) (layer "F.Cu") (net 10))
 (segment (start 48.7441 76.3684) (end 48.7441 101.6841) (width 0.2) (layer "F.Cu") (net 10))
 (segment (start 48.7441 101.6841) (end 50.31 103.25) (width 0.2) (layer "F.Cu") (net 10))
 (via (at 51.1188 73.9937) (size 0.6) (drill 0.3) (layers "F.Cu" "B.Cu") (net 10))
 (segment (start 77.1106 70.075) (end 74.4156 72.77) (width 0.2) (layer "B.Cu") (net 10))
 (segment (start 74.4156 72.77) (end 52.3425 72.77) (width 0.2) (layer "B.Cu") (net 10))
 (segment (start 97.5 71.18) (end 96.395 70.075) (width 0.2) (layer "B.Cu") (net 10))
 (segment (start 96.395 70.075) (end 77.1106 70.075) (width 0.2) (layer "B.Cu") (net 10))
 (segment (start 52.3425 72.77) (end 51.1188 73.9937) (width 0.2) (layer "B.Cu") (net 10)))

